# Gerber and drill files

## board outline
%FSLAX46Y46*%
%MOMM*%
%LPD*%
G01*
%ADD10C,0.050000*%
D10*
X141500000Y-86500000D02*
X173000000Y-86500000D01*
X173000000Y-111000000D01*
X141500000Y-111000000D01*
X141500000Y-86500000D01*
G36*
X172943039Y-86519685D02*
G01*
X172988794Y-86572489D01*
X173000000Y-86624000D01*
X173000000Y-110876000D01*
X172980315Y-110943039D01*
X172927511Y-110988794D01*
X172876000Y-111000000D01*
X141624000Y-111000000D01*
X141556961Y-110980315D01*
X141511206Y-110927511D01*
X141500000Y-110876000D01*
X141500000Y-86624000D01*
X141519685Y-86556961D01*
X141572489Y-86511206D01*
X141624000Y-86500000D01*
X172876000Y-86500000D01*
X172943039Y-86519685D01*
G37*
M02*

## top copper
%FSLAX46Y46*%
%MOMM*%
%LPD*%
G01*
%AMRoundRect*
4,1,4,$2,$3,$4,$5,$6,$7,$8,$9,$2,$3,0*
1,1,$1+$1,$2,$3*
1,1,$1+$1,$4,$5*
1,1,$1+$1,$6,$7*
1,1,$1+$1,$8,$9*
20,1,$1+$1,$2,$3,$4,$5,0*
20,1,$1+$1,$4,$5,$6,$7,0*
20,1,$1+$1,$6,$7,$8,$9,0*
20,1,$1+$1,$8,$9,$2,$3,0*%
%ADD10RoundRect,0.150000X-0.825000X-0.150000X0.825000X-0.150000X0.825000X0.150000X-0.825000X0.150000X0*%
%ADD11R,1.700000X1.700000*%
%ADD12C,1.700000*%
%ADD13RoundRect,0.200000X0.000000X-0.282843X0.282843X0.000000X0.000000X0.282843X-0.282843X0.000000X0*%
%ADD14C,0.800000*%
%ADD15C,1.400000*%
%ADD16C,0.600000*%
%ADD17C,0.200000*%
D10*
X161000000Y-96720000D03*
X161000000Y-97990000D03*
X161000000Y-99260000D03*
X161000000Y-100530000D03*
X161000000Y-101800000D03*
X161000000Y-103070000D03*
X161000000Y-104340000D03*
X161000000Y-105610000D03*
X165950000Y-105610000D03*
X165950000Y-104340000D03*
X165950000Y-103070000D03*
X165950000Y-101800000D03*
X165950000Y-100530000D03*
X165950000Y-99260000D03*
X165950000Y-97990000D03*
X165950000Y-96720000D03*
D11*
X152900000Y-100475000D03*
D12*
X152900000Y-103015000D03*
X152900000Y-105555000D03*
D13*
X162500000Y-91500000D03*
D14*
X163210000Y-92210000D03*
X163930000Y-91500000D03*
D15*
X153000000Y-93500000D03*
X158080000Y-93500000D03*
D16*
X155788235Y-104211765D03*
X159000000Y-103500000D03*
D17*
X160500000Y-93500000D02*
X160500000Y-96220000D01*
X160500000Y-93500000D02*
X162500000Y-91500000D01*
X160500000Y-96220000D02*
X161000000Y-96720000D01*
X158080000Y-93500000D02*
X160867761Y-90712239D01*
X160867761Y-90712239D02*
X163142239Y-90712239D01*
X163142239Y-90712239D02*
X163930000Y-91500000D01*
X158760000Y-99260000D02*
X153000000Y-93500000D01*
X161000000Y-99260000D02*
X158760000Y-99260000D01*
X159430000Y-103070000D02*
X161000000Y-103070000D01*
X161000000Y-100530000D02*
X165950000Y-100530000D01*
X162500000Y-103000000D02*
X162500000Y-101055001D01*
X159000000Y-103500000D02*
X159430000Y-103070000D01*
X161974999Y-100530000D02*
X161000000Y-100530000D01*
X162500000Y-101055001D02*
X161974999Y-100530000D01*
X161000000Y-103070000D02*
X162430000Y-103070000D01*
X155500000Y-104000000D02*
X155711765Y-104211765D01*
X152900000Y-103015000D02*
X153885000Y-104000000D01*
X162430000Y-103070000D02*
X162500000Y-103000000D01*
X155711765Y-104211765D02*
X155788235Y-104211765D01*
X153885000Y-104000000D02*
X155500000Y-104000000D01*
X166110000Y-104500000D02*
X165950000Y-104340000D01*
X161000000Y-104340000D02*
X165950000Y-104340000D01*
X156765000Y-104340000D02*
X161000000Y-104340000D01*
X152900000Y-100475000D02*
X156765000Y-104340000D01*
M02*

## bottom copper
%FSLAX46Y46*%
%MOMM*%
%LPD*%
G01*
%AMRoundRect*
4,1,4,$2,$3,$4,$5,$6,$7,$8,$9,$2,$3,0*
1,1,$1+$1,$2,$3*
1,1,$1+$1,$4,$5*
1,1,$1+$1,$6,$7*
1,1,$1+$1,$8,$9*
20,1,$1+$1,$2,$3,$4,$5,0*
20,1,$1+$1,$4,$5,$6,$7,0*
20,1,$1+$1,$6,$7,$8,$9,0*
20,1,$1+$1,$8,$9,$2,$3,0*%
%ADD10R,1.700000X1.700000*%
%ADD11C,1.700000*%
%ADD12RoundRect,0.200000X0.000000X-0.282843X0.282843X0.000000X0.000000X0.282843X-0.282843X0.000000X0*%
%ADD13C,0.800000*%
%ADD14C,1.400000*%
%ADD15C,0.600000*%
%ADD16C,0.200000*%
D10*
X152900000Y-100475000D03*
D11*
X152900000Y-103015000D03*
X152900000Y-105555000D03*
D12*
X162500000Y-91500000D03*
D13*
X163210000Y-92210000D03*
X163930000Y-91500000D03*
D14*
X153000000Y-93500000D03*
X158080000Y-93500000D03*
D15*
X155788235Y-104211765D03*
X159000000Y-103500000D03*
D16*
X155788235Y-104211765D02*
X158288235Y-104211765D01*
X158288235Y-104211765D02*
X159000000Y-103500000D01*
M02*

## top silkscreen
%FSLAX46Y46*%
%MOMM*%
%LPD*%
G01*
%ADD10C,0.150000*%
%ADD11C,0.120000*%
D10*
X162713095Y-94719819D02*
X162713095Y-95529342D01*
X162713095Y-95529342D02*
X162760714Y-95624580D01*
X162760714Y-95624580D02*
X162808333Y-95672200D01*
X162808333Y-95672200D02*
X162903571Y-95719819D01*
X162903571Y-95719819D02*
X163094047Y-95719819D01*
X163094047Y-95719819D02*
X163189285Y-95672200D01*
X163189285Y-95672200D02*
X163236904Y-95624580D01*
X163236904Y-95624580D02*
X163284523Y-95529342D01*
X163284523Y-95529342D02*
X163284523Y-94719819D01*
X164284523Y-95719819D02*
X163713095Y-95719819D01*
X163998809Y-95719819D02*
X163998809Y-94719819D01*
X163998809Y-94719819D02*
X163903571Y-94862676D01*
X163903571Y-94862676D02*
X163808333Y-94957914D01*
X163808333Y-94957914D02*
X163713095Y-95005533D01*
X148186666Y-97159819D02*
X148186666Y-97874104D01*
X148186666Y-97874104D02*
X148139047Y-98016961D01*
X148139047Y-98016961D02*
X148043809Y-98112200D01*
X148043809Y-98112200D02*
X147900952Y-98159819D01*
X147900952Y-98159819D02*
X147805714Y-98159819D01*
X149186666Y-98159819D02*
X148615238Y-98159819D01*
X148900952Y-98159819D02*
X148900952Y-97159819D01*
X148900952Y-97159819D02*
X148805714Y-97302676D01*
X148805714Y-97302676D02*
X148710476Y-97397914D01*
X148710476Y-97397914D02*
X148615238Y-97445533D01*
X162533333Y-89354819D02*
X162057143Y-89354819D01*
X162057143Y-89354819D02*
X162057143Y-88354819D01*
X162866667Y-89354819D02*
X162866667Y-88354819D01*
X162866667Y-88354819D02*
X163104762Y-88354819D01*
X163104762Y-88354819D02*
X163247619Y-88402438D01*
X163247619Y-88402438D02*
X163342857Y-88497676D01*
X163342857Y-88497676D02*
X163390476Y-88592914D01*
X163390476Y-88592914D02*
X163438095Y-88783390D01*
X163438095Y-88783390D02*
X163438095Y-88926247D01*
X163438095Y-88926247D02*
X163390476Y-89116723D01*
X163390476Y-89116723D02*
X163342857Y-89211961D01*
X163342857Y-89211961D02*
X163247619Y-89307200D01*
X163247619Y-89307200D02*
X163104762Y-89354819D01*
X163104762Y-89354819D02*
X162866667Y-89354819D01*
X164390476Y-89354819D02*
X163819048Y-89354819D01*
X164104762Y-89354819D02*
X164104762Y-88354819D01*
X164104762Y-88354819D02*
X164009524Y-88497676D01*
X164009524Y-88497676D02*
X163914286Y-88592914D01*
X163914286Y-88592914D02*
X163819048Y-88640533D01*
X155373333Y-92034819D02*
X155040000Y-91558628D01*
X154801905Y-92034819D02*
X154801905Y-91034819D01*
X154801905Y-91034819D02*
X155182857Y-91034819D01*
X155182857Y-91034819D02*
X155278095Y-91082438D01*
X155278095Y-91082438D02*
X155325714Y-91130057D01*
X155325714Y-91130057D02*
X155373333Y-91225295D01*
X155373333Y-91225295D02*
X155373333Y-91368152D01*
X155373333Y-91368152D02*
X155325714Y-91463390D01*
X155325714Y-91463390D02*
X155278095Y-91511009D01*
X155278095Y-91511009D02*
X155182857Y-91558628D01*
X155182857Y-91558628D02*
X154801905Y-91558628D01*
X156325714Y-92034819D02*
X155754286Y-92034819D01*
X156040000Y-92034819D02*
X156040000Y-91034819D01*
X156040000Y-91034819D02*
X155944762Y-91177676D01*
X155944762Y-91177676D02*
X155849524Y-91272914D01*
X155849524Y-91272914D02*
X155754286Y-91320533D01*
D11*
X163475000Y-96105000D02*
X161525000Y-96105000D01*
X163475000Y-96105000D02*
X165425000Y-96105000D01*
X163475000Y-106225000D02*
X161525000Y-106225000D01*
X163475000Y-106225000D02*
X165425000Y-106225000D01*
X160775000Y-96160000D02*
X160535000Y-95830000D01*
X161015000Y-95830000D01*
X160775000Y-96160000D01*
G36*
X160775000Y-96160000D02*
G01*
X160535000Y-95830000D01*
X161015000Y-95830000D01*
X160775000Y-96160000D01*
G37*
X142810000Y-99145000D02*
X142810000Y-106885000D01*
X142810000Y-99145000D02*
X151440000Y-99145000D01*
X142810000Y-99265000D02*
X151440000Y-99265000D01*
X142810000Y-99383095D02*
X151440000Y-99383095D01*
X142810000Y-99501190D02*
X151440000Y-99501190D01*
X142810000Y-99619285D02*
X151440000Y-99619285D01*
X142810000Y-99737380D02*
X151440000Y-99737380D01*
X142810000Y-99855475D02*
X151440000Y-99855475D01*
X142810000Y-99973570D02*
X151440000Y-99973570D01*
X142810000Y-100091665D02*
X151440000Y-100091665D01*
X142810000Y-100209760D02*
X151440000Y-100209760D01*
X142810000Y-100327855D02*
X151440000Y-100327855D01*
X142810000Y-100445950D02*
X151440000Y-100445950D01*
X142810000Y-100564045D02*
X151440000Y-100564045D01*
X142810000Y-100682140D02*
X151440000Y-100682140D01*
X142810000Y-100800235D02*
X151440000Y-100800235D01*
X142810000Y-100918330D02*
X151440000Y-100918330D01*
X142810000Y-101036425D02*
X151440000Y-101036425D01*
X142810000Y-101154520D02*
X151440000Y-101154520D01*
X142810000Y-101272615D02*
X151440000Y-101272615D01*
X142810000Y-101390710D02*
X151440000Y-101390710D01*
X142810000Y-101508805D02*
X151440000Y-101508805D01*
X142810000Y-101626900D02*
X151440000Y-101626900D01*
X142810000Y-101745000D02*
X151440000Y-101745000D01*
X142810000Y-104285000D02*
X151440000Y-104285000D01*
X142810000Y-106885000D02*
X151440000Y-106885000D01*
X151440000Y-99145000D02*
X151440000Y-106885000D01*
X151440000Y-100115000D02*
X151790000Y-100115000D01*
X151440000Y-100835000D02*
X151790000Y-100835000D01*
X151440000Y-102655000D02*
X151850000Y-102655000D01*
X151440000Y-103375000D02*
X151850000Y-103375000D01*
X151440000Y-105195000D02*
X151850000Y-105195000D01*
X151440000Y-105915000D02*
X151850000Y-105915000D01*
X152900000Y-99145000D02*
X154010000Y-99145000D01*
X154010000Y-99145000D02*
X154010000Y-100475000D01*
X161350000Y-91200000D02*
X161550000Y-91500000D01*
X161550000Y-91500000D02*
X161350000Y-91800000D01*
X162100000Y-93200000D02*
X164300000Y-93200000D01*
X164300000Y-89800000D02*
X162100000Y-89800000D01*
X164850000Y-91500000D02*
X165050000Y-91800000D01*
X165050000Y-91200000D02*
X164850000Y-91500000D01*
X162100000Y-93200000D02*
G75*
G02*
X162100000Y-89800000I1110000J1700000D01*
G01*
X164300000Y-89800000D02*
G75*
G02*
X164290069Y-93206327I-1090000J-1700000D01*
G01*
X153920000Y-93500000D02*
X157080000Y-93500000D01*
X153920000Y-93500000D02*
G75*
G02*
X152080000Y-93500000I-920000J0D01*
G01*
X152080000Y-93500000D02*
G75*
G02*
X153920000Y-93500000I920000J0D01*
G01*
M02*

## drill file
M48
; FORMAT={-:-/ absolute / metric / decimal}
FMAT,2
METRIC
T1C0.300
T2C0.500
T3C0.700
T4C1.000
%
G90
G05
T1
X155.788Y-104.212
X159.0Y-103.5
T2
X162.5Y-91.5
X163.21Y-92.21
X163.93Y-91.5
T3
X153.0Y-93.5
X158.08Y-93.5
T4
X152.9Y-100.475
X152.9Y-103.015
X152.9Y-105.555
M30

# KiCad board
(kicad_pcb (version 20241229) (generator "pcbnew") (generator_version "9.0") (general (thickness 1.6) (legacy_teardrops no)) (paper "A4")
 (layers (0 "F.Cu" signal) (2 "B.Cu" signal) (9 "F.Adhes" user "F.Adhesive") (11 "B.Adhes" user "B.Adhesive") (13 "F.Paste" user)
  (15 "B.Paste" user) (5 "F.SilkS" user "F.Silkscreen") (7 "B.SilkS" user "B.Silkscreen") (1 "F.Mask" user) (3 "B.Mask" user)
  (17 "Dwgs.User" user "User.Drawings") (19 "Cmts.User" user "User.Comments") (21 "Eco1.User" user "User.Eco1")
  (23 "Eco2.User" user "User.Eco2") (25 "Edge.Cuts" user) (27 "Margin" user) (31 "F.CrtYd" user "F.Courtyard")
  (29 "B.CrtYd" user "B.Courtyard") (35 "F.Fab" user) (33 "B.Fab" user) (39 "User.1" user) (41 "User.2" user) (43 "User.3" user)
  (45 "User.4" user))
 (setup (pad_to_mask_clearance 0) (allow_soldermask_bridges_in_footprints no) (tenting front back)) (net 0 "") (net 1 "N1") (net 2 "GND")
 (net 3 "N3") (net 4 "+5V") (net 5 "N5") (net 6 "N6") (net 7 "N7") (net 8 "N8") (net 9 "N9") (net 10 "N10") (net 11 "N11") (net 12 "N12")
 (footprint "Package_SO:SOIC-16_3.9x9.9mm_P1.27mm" (layer "F.Cu") (at 163.475 101.165)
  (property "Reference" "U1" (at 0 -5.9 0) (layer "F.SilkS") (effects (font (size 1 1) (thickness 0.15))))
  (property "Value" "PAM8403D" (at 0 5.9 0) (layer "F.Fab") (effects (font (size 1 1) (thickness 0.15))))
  (fp_line (start 0 -5.06) (end -1.95 -5.06) (stroke (width 0.12) (type solid)) (layer "F.SilkS"))
  (fp_line (start 0 -5.06) (end 1.95 -5.06) (stroke (width 0.12) (type solid)) (layer "F.SilkS"))
  (fp_line (start 0 5.06) (end -1.95 5.06) (stroke (width 0.12) (type solid)) (layer "F.SilkS"))
  (fp_line (start 0 5.06) (end 1.95 5.06) (stroke (width 0.12) (type solid)) (layer "F.SilkS"))
  (fp_poly (pts (xy -2.7 -5.005) (xy -2.94 -5.335) (xy -2.46 -5.335)) (stroke (width 0.12) (type solid)) (fill yes) (layer "F.SilkS"))
  (pad "1" smd roundrect (at -2.475 -4.445) (size 1.95 0.6) (layers "F.Cu" "F.Mask" "F.Paste") (roundrect_rratio 0.25) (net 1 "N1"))
  (pad "2" smd roundrect (at -2.475 -3.175) (size 1.95 0.6) (layers "F.Cu" "F.Mask" "F.Paste") (roundrect_rratio 0.25) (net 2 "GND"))
  (pad "3" smd roundrect (at -2.475 -1.905) (size 1.95 0.6) (layers "F.Cu" "F.Mask" "F.Paste") (roundrect_rratio 0.25) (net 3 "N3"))
  (pad "4" smd roundrect (at -2.475 -0.635) (size 1.95 0.6) (layers "F.Cu" "F.Mask" "F.Paste") (roundrect_rratio 0.25) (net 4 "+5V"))
  (pad "5" smd roundrect (at -2.475 0.635) (size 1.95 0.6) (layers "F.Cu" "F.Mask" "F.Paste") (roundrect_rratio 0.25) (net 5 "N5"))
  (pad "6" smd roundrect (at -2.475 1.905) (size 1.95 0.6) (layers "F.Cu" "F.Mask" "F.Paste") (roundrect_rratio 0.25) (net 4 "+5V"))
  (pad "7" smd roundrect (at -2.475 3.175) (size 1.95 0.6) (layers "F.Cu" "F.Mask" "F.Paste") (roundrect_rratio 0.25) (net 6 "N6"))
  (pad "8" smd roundrect (at -2.475 4.445) (size 1.95 0.6) (layers "F.Cu" "F.Mask" "F.Paste") (roundrect_rratio 0.25) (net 2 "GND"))
  (pad "9" smd roundrect (at 2.475 4.445) (size 1.95 0.6) (layers "F.Cu" "F.Mask" "F.Paste") (roundrect_rratio 0.25) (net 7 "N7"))
  (pad "10" smd roundrect (at 2.475 3.175) (size 1.95 0.6) (layers "F.Cu" "F.Mask" "F.Paste") (roundrect_rratio 0.25) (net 6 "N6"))
  (pad "11" smd roundrect (at 2.475 1.905) (size 1.95 0.6) (layers "F.Cu" "F.Mask" "F.Paste") (roundrect_rratio 0.25) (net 2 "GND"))
  (pad "12" smd roundrect (at 2.475 0.635) (size 1.95 0.6) (layers "F.Cu" "F.Mask" "F.Paste") (roundrect_rratio 0.25) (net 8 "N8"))
  (pad "13" smd roundrect (at 2.475 -0.635) (size 1.95 0.6) (layers "F.Cu" "F.Mask" "F.Paste") (roundrect_rratio 0.25) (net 4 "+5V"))
  (pad "14" smd roundrect (at 2.475 -1.905) (size 1.95 0.6) (layers "F.Cu" "F.Mask" "F.Paste") (roundrect_rratio 0.25) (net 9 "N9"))
  (pad "15" smd roundrect (at 2.475 -3.175) (size 1.95 0.6) (layers "F.Cu" "F.Mask" "F.Paste") (roundrect_rratio 0.25) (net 2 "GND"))
  (pad "16" smd roundrect (at 2.475 -4.445) (size 1.95 0.6) (layers "F.Cu" "F.Mask" "F.Paste") (roundrect_rratio 0.25) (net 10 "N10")))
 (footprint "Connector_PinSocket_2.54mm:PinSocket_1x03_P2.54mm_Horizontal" (layer "F.Cu") (at 152.9 100.475)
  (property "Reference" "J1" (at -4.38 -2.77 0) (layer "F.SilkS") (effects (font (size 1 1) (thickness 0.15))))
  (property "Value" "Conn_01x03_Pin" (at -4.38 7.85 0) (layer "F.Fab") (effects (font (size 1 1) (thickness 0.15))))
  (fp_line (start -10.09 -1.33) (end -10.09 6.41) (stroke (width 0.12) (type solid)) (layer "F.SilkS"))
  (fp_line (start -10.09 -1.33) (end -1.46 -1.33) (stroke (width 0.12) (type solid)) (layer "F.SilkS"))
  (fp_line (start -10.09 -1.21) (end -1.46 -1.21) (stroke (width 0.12) (type solid)) (layer "F.SilkS"))
  (fp_line (start -10.09 -1.091905) (end -1.46 -1.091905) (stroke (width 0.12) (type solid)) (layer "F.SilkS"))
  (fp_line (start -10.09 -0.97381) (end -1.46 -0.97381) (stroke (width 0.12) (type solid)) (layer "F.SilkS"))
  (fp_line (start -10.09 -0.855715) (end -1.46 -0.855715) (stroke (width 0.12) (type solid)) (layer "F.SilkS"))
  (fp_line (start -10.09 -0.73762) (end -1.46 -0.73762) (stroke (width 0.12) (type solid)) (layer "F.SilkS"))
  (fp_line (start -10.09 -0.619525) (end -1.46 -0.619525) (stroke (width 0.12) (type solid)) (layer "F.SilkS"))
  (fp_line (start -10.09 -0.50143) (end -1.46 -0.50143) (stroke (width 0.12) (type solid)) (layer "F.SilkS"))
  (fp_line (start -10.09 -0.383335) (end -1.46 -0.383335) (stroke (width 0.12) (type solid)) (layer "F.SilkS"))
  (fp_line (start -10.09 -0.26524) (end -1.46 -0.26524) (stroke (width 0.12) (type solid)) (layer "F.SilkS"))
  (fp_line (start -10.09 -0.147145) (end -1.46 -0.147145) (stroke (width 0.12) (type solid)) (layer "F.SilkS"))
  (fp_line (start -10.09 -0.02905) (end -1.46 -0.02905) (stroke (width 0.12) (type solid)) (layer "F.SilkS"))
  (fp_line (start -10.09 0.089045) (end -1.46 0.089045) (stroke (width 0.12) (type solid)) (layer "F.SilkS"))
  (fp_line (start -10.09 0.20714) (end -1.46 0.20714) (stroke (width 0.12) (type solid)) (layer "F.SilkS"))
  (fp_line (start -10.09 0.325235) (end -1.46 0.325235) (stroke (width 0.12) (type solid)) (layer "F.SilkS"))
  (fp_line (start -10.09 0.44333) (end -1.46 0.44333) (stroke (width 0.12) (type solid)) (layer "F.SilkS"))
  (fp_line (start -10.09 0.561425) (end -1.46 0.561425) (stroke (width 0.12) (type solid)) (layer "F.SilkS"))
  (fp_line (start -10.09 0.67952) (end -1.46 0.67952) (stroke (width 0.12) (type solid)) (layer "F.SilkS"))
  (fp_line (start -10.09 0.797615) (end -1.46 0.797615) (stroke (width 0.12) (type solid)) (layer "F.SilkS"))
  (fp_line (start -10.09 0.91571) (end -1.46 0.91571) (stroke (width 0.12) (type solid)) (layer "F.SilkS"))
  (fp_line (start -10.09 1.033805) (end -1.46 1.033805) (stroke (width 0.12) (type solid)) (layer "F.SilkS"))
  (fp_line (start -10.09 1.1519) (end -1.46 1.1519) (stroke (width 0.12) (type solid)) (layer "F.SilkS"))
  (fp_line (start -10.09 1.27) (end -1.46 1.27) (stroke (width 0.12) (type solid)) (layer "F.SilkS"))
  (fp_line (start -10.09 3.81) (end -1.46 3.81) (stroke (width 0.12) (type solid)) (layer "F.SilkS"))
  (fp_line (start -10.09 6.41) (end -1.46 6.41) (stroke (width 0.12) (type solid)) (layer "F.SilkS"))
  (fp_line (start -1.46 -1.33) (end -1.46 6.41) (stroke (width 0.12) (type solid)) (layer "F.SilkS"))
  (fp_line (start -1.46 -0.36) (end -1.11 -0.36) (stroke (width 0.12) (type solid)) (layer "F.SilkS"))
  (fp_line (start -1.46 0.36) (end -1.11 0.36) (stroke (width 0.12) (type solid)) (layer "F.SilkS"))
  (fp_line (start -1.46 2.18) (end -1.05 2.18) (stroke (width 0.12) (type solid)) (layer "F.SilkS"))
  (fp_line (start -1.46 2.9) (end -1.05 2.9) (stroke (width 0.12) (type solid)) (layer "F.SilkS"))
  (fp_line (start -1.46 4.72) (end -1.05 4.72) (stroke (width 0.12) (type solid)) (layer "F.SilkS"))
  (fp_line (start -1.46 5.44) (end -1.05 5.44) (stroke (width 0.12) (type solid)) (layer "F.SilkS"))
  (fp_line (start 0 -1.33) (end 1.11 -1.33) (stroke (width 0.12) (type solid)) (layer "F.SilkS"))
  (fp_line (start 1.11 -1.33) (end 1.11 0) (stroke (width 0.12) (type solid)) (layer "F.SilkS"))
  (pad "1" thru_hole rect (at 0 0) (size 1.7 1.7) (drill 1) (layers "*.Cu" "*.Mask") (remove_unused_layers no) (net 6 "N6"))
  (pad "2" thru_hole circle (at 0 2.54) (size 1.7 1.7) (drill 1) (layers "*.Cu" "*.Mask") (remove_unused_layers no) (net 4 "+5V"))
  (pad "3" thru_hole circle (at 0 5.08) (size 1.7 1.7) (drill 1) (layers "*.Cu" "*.Mask") (remove_unused_layers no) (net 2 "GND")))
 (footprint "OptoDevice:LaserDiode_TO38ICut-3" (layer "F.Cu") (at 162.5 91.5)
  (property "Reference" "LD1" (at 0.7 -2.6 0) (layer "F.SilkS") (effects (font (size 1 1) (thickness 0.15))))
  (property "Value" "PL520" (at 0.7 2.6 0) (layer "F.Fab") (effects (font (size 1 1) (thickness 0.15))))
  (fp_line (start -1.15 -0.3) (end -0.95 0) (stroke (width 0.12) (type solid)) (layer "F.SilkS"))
  (fp_line (start -0.95 0) (end -1.15 0.3) (stroke (width 0.12) (type solid)) (layer "F.SilkS"))
  (fp_line (start -0.4 1.7) (end 1.8 1.7) (stroke (width 0.12) (type solid)) (layer "F.SilkS"))
  (fp_line (start 1.8 -1.7) (end -0.4 -1.7) (stroke (width 0.12) (type solid)) (layer "F.SilkS"))
  (fp_line (start 2.35 0) (end 2.55 0.3) (stroke (width 0.12) (type solid)) (layer "F.SilkS"))
  (fp_line (start 2.55 -0.3) (end 2.35 0) (stroke (width 0.12) (type solid)) (layer "F.SilkS"))
  (fp_arc (start -0.4 1.7) (mid -1.320296 0) (end -0.4 -1.7) (stroke (width 0.12) (type solid)) (layer "F.SilkS"))
  (fp_arc (start 1.8 -1.7) (mid 2.729422 0.005888) (end 1.790069 1.706327) (stroke (width 0.12) (type solid)) (layer "F.SilkS"))
  (pad "1" thru_hole roundrect (at 0 0 45) (size 0.8 0.8) (drill 0.5) (layers "*.Cu" "*.Mask") (remove_unused_layers no)
   (roundrect_rratio 0.25) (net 1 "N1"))
  (pad "2" thru_hole circle (at 0.71 0.71) (size 0.8 0.8) (drill 0.5) (layers "*.Cu" "*.Mask") (remove_unused_layers no) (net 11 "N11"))
  (pad "3" thru_hole circle (at 1.43 0) (size 0.8 0.8) (drill 0.5) (layers "*.Cu" "*.Mask") (remove_unused_layers no) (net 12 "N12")))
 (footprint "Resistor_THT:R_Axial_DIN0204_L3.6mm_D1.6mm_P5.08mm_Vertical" (layer "F.Cu") (at 153 93.5)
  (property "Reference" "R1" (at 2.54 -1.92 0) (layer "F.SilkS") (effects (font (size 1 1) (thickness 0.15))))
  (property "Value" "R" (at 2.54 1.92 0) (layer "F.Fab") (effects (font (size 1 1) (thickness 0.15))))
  (fp_line (start 0.92 0) (end 4.08 0) (stroke (width 0.12) (type solid)) (layer "F.SilkS"))
  (fp_circle (center 0 0) (end 0.92 0) (stroke (width 0.12) (type solid)) (fill no) (layer "F.SilkS"))
  (pad "1" thru_hole circle (at 0 0) (size 1.4 1.4) (drill 0.7) (layers "*.Cu" "*.Mask") (remove_unused_layers no) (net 3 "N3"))
  (pad "2" thru_hole circle (at 5.08 0) (size 1.4 1.4) (drill 0.7) (layers "*.Cu" "*.Mask") (remove_unused_layers no) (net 12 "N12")))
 (gr_rect (start 141.5 86.5) (end 173 111) (stroke (width 0.05) (type default)) (fill no) (layer "Edge.Cuts"))
 (segment (start 160.5 93.5) (end 160.5 96.22) (width 0.2) (layer "F.Cu") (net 1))
 (segment (start 160.5 93.5) (end 162.5 91.5) (width 0.2) (layer "F.Cu") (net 1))
 (segment (start 160.5 96.22) (end 161 96.72) (width 0.2) (layer "F.Cu") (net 1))
 (segment (start 158.08 93.5) (end 160.867761 90.712239) (width 0.2) (layer "F.Cu") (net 12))
 (segment (start 160.867761 90.712239) (end 163.142239 90.712239) (width 0.2) (layer "F.Cu") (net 12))
 (segment (start 163.142239 90.712239) (end 163.93 91.5) (width 0.2) (layer "F.Cu") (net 12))
 (segment (start 158.76 99.26) (end 153 93.5) (width 0.2) (layer "F.Cu") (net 3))
 (segment (start 161 99.26) (end 158.76 99.26) (width 0.2) (layer "F.Cu") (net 3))
 (segment (start 159.43 103.07) (end 161 103.07) (width 0.2) (layer "F.Cu") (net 4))
 (segment (start 161 100.53) (end 165.95 100.53) (width 0.2) (layer "F.Cu") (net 4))
 (segment (start 162.5 103) (end 162.5 101.055001) (width 0.2) (layer "F.Cu") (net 4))
 (segment (start 159 103.5) (end 159.43 103.07) (width 0.2) (layer "F.Cu") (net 4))
 (segment (start 161.974999 100.53) (end 161 100.53) (width 0.2) (layer "F.Cu") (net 4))
 (segment (start 162.5 101.055001) (end 161.974999 100.53) (width 0.2) (layer "F.Cu") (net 4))
 (segment (start 161 103.07) (end 162.43 103.07) (width 0.2) (layer "F.Cu") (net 4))
 (segment (start 155.5 104) (end 155.711765 104.211765) (width 0.2) (layer "F.Cu") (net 4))
 (segment (start 152.9 103.015) (end 153.885 104) (width 0.2) (layer "F.Cu") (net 4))
 (segment (start 162.43 103.07) (end 162.5 103) (width 0.2) (layer "F.Cu") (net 4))
 (segment (start 155.711765 104.211765) (end 155.788235 104.211765) (width 0.2) (layer "F.Cu") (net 4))
 (segment (start 153.885 104) (end 155.5 104) (width 0.2) (layer "F.Cu") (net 4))
 (via (at 155.788235 104.211765) (size 0.6) (drill 0.3) (layers "F.Cu" "B.Cu") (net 4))
 (via (at 159 103.5) (size 0.6) (drill 0.3) (layers "F.Cu" "B.Cu") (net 4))
 (segment (start 155.788235 104.211765) (end 158.288235 104.211765) (width 0.2) (layer "B.Cu") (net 4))
 (segment (start 158.288235 104.211765) (end 159 103.5) (width 0.2) (layer "B.Cu") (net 4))
 (segment (start 166.11 104.5) (end 165.95 104.34) (width 0.2) (layer "F.Cu") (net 6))
 (segment (start 161 104.34) (end 165.95 104.34) (width 0.2) (layer "F.Cu") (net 6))
 (segment (start 156.765 104.34) (end 161 104.34) (width 0.2) (layer "F.Cu") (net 6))
 (segment (start 152.9 100.475) (end 156.765 104.34) (width 0.2) (layer "F.Cu") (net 6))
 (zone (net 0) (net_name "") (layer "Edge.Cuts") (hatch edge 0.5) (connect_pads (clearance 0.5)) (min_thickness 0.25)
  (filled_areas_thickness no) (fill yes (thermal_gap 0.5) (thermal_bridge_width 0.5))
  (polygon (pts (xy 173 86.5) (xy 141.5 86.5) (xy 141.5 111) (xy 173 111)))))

